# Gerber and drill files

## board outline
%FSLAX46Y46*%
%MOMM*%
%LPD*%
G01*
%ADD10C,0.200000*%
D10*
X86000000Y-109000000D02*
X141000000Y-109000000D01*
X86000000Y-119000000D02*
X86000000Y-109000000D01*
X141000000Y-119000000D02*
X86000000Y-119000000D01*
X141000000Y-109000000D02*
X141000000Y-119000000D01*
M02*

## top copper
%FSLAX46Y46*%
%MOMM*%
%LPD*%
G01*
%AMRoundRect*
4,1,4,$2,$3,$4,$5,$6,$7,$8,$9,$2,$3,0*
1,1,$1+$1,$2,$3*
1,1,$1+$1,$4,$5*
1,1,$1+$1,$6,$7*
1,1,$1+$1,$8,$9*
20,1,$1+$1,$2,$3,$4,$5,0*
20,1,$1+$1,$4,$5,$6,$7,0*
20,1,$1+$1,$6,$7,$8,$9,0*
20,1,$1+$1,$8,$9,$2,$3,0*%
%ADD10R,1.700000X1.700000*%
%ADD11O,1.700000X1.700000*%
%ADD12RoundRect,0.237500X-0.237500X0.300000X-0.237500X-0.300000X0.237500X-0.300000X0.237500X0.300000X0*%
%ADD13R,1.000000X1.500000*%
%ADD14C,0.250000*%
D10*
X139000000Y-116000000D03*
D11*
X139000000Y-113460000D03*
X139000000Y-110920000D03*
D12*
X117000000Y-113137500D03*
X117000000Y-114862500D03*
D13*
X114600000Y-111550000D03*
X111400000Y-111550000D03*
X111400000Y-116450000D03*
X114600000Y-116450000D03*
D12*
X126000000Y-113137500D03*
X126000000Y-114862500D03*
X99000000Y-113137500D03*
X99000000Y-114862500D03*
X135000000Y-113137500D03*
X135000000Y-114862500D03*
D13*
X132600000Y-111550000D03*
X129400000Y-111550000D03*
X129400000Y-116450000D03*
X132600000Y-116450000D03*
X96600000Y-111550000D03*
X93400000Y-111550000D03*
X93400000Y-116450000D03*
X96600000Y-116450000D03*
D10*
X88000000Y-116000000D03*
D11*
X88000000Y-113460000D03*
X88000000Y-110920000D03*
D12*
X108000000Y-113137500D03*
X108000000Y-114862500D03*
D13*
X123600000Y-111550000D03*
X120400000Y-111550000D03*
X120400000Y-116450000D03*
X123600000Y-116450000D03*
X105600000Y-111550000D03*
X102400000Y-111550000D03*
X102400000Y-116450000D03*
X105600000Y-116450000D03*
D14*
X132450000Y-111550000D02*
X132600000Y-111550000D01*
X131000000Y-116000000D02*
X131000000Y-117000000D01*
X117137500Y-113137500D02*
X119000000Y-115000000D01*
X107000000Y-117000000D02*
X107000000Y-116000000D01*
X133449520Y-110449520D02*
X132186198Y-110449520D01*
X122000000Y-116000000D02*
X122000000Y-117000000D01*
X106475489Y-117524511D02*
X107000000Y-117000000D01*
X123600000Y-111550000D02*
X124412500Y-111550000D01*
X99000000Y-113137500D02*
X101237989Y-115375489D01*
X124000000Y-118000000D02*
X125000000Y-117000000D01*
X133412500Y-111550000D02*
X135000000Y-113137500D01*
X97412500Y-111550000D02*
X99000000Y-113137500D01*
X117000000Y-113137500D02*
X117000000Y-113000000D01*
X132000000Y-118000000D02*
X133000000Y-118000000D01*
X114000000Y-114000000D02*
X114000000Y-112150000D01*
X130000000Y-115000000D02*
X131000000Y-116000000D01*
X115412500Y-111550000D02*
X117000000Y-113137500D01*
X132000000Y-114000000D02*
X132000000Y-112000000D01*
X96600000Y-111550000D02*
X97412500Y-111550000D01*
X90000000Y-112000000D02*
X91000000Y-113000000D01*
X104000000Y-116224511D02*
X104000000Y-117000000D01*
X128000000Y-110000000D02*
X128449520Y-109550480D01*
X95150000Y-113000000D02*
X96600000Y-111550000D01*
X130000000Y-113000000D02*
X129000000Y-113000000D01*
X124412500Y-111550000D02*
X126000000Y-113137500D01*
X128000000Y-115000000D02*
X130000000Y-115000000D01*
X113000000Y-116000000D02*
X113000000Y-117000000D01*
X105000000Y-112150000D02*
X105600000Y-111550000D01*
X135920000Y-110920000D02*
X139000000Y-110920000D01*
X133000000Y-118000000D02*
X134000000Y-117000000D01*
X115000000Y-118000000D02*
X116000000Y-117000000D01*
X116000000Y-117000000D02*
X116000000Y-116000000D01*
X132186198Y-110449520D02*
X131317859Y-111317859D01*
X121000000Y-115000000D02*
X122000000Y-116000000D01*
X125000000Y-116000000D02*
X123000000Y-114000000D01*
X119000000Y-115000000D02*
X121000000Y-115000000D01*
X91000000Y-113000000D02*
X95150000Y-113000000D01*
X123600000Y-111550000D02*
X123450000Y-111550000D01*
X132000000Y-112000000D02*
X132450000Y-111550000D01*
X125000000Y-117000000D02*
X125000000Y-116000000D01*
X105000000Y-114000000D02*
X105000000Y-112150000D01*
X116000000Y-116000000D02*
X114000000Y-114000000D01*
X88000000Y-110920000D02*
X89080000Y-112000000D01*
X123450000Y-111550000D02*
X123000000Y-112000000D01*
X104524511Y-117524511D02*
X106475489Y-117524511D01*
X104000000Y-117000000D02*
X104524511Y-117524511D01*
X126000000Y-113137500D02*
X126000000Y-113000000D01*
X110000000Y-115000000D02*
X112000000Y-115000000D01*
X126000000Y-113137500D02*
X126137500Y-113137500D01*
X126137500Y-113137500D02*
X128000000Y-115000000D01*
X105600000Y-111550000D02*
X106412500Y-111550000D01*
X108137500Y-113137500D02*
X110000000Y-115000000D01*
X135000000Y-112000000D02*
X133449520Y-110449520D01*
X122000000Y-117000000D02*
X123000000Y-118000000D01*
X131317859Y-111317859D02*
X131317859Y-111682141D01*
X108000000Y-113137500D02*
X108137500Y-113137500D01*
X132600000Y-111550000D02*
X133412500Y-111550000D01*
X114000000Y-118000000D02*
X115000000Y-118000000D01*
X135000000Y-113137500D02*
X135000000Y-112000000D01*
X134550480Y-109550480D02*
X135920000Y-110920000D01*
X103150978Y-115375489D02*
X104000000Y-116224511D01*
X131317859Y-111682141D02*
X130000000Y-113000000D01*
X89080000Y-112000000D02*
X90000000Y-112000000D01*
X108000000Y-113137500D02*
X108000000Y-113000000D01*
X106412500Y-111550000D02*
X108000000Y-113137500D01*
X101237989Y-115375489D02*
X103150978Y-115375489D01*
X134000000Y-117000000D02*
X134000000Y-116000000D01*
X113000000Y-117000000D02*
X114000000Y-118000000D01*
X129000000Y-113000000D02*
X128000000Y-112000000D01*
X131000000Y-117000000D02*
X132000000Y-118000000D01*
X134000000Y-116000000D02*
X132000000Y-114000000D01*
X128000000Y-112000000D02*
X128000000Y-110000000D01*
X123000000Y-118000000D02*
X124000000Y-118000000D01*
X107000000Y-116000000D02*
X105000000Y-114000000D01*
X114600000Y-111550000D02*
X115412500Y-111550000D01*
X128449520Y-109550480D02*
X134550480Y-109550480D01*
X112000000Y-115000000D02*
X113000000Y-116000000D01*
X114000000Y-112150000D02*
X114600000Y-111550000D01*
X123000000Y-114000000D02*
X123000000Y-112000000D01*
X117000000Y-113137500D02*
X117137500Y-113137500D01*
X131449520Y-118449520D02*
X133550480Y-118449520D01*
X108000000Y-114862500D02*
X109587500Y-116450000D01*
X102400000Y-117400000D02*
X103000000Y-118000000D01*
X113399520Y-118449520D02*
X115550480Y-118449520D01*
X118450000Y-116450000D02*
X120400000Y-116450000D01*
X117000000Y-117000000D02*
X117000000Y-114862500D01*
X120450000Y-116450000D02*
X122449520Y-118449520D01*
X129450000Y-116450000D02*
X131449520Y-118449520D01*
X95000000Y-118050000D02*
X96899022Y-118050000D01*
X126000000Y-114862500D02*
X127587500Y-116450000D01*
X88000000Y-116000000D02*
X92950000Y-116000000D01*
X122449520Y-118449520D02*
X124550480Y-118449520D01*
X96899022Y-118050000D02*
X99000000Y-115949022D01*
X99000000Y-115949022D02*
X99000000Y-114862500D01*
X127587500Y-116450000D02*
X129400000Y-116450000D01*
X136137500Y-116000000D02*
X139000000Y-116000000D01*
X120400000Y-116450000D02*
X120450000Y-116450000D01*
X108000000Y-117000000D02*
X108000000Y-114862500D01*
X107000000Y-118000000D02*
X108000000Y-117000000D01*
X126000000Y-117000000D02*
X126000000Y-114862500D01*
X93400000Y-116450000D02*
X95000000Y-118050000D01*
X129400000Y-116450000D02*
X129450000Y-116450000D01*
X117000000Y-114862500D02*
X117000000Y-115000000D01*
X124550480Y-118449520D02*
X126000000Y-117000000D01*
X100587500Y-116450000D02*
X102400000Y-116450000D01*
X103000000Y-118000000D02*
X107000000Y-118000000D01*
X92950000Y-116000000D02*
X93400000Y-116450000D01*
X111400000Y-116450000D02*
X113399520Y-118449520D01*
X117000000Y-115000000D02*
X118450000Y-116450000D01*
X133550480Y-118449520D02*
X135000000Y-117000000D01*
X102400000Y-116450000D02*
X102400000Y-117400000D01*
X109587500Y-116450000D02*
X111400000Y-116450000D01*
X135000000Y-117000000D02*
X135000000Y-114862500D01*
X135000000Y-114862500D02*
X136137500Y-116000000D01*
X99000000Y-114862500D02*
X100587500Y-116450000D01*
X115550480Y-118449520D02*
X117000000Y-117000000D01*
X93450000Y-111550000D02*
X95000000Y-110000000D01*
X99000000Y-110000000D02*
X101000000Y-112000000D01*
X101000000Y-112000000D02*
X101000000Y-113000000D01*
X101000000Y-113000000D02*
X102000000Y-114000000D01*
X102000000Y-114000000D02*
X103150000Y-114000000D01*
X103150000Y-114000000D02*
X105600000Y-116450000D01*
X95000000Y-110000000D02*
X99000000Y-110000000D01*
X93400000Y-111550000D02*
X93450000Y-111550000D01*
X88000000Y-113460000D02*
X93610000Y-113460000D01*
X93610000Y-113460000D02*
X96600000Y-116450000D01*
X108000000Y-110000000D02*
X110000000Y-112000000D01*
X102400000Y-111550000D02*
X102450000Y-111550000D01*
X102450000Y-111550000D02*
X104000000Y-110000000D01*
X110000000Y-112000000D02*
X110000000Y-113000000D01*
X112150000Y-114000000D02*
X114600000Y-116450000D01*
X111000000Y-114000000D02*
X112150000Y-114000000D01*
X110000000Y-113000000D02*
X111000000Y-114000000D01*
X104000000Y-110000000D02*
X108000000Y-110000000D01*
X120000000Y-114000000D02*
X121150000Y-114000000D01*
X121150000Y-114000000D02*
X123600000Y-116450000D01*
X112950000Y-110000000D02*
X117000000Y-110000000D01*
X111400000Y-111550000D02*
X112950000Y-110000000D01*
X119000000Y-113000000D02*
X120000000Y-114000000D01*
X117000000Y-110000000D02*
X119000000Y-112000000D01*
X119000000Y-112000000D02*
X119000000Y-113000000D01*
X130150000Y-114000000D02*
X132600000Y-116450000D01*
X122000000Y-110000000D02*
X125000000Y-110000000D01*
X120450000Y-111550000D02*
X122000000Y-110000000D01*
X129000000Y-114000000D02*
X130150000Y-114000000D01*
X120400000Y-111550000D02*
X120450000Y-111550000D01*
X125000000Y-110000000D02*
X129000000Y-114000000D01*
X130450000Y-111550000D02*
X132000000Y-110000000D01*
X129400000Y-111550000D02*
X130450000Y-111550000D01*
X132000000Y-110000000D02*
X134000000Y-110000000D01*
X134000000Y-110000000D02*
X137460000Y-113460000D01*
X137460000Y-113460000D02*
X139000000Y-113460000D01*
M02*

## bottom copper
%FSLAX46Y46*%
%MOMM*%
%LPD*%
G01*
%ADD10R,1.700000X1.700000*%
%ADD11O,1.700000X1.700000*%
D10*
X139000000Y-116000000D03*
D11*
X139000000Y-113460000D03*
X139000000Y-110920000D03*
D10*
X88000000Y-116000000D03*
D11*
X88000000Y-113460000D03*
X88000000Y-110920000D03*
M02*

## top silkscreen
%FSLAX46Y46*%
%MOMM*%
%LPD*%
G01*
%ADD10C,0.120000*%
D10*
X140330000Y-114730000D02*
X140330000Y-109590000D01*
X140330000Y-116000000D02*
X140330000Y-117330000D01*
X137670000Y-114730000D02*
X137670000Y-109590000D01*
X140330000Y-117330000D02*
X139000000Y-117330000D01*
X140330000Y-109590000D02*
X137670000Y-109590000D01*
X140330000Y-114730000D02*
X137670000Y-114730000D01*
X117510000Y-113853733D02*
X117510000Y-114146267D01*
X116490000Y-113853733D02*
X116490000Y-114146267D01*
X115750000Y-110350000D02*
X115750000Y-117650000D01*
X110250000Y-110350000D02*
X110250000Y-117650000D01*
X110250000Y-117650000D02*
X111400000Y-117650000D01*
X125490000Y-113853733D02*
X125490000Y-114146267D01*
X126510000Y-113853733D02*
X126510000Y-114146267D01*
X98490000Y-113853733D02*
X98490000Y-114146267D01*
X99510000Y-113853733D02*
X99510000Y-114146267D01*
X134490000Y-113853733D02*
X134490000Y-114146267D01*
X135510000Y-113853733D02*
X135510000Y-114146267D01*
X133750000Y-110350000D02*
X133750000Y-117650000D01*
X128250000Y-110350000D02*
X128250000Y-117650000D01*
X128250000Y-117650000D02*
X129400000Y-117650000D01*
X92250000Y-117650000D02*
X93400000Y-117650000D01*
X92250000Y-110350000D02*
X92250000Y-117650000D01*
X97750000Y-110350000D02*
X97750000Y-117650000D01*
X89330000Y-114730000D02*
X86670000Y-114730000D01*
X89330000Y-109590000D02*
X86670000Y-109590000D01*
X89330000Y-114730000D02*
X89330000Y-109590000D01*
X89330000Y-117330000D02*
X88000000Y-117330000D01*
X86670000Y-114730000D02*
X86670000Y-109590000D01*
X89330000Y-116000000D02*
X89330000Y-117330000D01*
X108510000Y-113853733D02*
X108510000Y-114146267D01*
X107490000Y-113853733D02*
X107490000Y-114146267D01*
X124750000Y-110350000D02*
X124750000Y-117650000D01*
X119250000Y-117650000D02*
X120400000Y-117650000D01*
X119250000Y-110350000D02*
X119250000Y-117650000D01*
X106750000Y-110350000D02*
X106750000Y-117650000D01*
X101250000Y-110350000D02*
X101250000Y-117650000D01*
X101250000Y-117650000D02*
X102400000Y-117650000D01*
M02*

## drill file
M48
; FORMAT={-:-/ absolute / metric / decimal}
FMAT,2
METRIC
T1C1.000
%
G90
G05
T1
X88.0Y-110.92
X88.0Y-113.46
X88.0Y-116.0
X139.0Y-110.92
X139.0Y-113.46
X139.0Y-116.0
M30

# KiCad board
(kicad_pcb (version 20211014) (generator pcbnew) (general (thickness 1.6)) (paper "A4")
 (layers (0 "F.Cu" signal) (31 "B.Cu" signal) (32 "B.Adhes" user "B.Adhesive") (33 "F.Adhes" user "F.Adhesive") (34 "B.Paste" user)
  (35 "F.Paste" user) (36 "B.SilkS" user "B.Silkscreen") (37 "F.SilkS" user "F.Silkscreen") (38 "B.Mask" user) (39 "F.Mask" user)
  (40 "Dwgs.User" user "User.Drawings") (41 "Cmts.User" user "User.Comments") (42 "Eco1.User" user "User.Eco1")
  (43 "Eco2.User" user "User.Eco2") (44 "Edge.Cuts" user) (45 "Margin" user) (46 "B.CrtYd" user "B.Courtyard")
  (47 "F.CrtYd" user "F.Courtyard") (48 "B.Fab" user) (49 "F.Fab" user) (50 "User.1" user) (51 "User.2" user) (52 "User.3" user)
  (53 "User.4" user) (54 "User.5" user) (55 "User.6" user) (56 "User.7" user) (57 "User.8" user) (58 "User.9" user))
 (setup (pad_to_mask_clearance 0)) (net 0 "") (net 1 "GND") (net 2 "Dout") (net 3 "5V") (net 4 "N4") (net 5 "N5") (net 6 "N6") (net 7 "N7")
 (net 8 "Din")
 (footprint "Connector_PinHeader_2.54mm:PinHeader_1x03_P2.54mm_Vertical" (layer "F.Cu") (at 139 116 180)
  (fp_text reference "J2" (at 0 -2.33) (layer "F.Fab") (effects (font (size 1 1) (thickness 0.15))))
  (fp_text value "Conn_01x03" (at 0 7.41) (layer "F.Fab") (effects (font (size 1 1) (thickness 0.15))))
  (fp_line (start -1.33 1.27) (end -1.33 6.41) (layer "F.SilkS") (width 0.12))
  (fp_line (start -1.33 0) (end -1.33 -1.33) (layer "F.SilkS") (width 0.12))
  (fp_line (start 1.33 1.27) (end 1.33 6.41) (layer "F.SilkS") (width 0.12))
  (fp_line (start -1.33 -1.33) (end 0 -1.33) (layer "F.SilkS") (width 0.12))
  (fp_line (start -1.33 6.41) (end 1.33 6.41) (layer "F.SilkS") (width 0.12))
  (fp_line (start -1.33 1.27) (end 1.33 1.27) (layer "F.SilkS") (width 0.12))
  (pad "1" thru_hole rect (at 0 0 180) (size 1.7 1.7) (drill 1) (layers *.Cu *.Mask) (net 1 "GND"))
  (pad "2" thru_hole oval (at 0 2.54 180) (size 1.7 1.7) (drill 1) (layers *.Cu *.Mask) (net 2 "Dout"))
  (pad "3" thru_hole oval (at 0 5.08 180) (size 1.7 1.7) (drill 1) (layers *.Cu *.Mask) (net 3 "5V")))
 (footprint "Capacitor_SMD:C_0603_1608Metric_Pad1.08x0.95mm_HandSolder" (layer "F.Cu") (at 117 114 -90)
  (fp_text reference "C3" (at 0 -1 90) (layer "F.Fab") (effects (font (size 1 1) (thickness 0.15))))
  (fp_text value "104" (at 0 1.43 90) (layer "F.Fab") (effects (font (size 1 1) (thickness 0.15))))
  (fp_line (start -0.146267 -0.51) (end 0.146267 -0.51) (layer "F.SilkS") (width 0.12))
  (fp_line (start -0.146267 0.51) (end 0.146267 0.51) (layer "F.SilkS") (width 0.12))
  (pad "1" smd roundrect (at -0.8625 0 270) (size 1.075 0.95) (layers "F.Cu" "F.Paste" "F.Mask") (roundrect_rratio 0.25) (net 3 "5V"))
  (pad "2" smd roundrect (at 0.8625 0 270) (size 1.075 0.95) (layers "F.Cu" "F.Paste" "F.Mask") (roundrect_rratio 0.25) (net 1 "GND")))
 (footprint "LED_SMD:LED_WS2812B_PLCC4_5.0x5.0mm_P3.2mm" (layer "F.Cu") (at 113 114 -90)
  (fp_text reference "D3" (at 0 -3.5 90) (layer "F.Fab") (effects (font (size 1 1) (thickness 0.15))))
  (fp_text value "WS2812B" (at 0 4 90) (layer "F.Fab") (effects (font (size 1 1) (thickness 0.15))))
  (fp_line (start -3.65 -2.75) (end 3.65 -2.75) (layer "F.SilkS") (width 0.12))
  (fp_line (start -3.65 2.75) (end 3.65 2.75) (layer "F.SilkS") (width 0.12))
  (fp_line (start 3.65 2.75) (end 3.65 1.6) (layer "F.SilkS") (width 0.12))
  (pad "1" smd rect (at -2.45 -1.6 270) (size 1.5 1) (layers "F.Cu" "F.Paste" "F.Mask") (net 3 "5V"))
  (pad "2" smd rect (at -2.45 1.6 270) (size 1.5 1) (layers "F.Cu" "F.Paste" "F.Mask") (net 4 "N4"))
  (pad "3" smd rect (at 2.45 1.6 270) (size 1.5 1) (layers "F.Cu" "F.Paste" "F.Mask") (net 1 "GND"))
  (pad "4" smd rect (at 2.45 -1.6 270) (size 1.5 1) (layers "F.Cu" "F.Paste" "F.Mask") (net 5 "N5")))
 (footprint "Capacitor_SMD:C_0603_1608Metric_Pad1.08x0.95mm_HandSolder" (layer "F.Cu") (at 126 114 -90)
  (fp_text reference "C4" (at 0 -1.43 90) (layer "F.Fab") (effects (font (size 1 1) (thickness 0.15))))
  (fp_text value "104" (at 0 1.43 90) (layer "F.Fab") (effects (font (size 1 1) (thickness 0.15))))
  (fp_line (start -0.146267 0.51) (end 0.146267 0.51) (layer "F.SilkS") (width 0.12))
  (fp_line (start -0.146267 -0.51) (end 0.146267 -0.51) (layer "F.SilkS") (width 0.12))
  (pad "1" smd roundrect (at -0.8625 0 270) (size 1.075 0.95) (layers "F.Cu" "F.Paste" "F.Mask") (roundrect_rratio 0.25) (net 3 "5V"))
  (pad "2" smd roundrect (at 0.8625 0 270) (size 1.075 0.95) (layers "F.Cu" "F.Paste" "F.Mask") (roundrect_rratio 0.25) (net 1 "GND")))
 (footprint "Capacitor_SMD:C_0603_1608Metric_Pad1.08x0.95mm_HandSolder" (layer "F.Cu") (at 99 114 -90)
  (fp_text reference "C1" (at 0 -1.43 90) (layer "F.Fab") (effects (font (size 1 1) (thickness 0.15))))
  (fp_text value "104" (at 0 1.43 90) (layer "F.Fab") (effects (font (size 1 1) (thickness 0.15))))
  (fp_line (start -0.146267 0.51) (end 0.146267 0.51) (layer "F.SilkS") (width 0.12))
  (fp_line (start -0.146267 -0.51) (end 0.146267 -0.51) (layer "F.SilkS") (width 0.12))
  (pad "1" smd roundrect (at -0.8625 0 270) (size 1.075 0.95) (layers "F.Cu" "F.Paste" "F.Mask") (roundrect_rratio 0.25) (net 3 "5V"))
  (pad "2" smd roundrect (at 0.8625 0 270) (size 1.075 0.95) (layers "F.Cu" "F.Paste" "F.Mask") (roundrect_rratio 0.25) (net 1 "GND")))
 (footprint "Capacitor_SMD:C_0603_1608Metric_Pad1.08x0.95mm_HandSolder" (layer "F.Cu") (at 135 114 -90)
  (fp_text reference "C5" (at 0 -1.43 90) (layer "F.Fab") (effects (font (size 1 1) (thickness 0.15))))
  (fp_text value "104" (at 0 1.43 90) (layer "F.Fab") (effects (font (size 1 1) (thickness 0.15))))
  (fp_line (start -0.146267 0.51) (end 0.146267 0.51) (layer "F.SilkS") (width 0.12))
  (fp_line (start -0.146267 -0.51) (end 0.146267 -0.51) (layer "F.SilkS") (width 0.12))
  (pad "1" smd roundrect (at -0.8625 0 270) (size 1.075 0.95) (layers "F.Cu" "F.Paste" "F.Mask") (roundrect_rratio 0.25) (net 3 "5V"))
  (pad "2" smd roundrect (at 0.8625 0 270) (size 1.075 0.95) (layers "F.Cu" "F.Paste" "F.Mask") (roundrect_rratio 0.25) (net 1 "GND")))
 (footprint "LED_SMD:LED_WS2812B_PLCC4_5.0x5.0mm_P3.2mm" (layer "F.Cu") (at 131 114 -90)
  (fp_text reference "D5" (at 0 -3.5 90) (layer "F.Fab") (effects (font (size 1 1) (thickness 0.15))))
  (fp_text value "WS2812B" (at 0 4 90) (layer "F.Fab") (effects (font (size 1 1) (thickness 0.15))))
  (fp_line (start -3.65 -2.75) (end 3.65 -2.75) (layer "F.SilkS") (width 0.12))
  (fp_line (start -3.65 2.75) (end 3.65 2.75) (layer "F.SilkS") (width 0.12))
  (fp_line (start 3.65 2.75) (end 3.65 1.6) (layer "F.SilkS") (width 0.12))
  (pad "1" smd rect (at -2.45 -1.6 270) (size 1.5 1) (layers "F.Cu" "F.Paste" "F.Mask") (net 3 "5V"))
  (pad "2" smd rect (at -2.45 1.6 270) (size 1.5 1) (layers "F.Cu" "F.Paste" "F.Mask") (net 2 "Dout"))
  (pad "3" smd rect (at 2.45 1.6 270) (size 1.5 1) (layers "F.Cu" "F.Paste" "F.Mask") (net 1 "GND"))
  (pad "4" smd rect (at 2.45 -1.6 270) (size 1.5 1) (layers "F.Cu" "F.Paste" "F.Mask") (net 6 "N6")))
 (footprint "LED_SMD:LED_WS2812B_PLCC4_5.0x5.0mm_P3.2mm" (layer "F.Cu") (at 95 114 -90)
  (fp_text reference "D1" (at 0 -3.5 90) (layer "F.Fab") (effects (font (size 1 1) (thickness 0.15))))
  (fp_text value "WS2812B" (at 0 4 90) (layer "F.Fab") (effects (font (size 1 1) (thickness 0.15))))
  (fp_line (start 3.65 2.75) (end 3.65 1.6) (layer "F.SilkS") (width 0.12))
  (fp_line (start -3.65 2.75) (end 3.65 2.75) (layer "F.SilkS") (width 0.12))
  (fp_line (start -3.65 -2.75) (end 3.65 -2.75) (layer "F.SilkS") (width 0.12))
  (pad "1" smd rect (at -2.45 -1.6 270) (size 1.5 1) (layers "F.Cu" "F.Paste" "F.Mask") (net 3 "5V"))
  (pad "2" smd rect (at -2.45 1.6 270) (size 1.5 1) (layers "F.Cu" "F.Paste" "F.Mask") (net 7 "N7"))
  (pad "3" smd rect (at 2.45 1.6 270) (size 1.5 1) (layers "F.Cu" "F.Paste" "F.Mask") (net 1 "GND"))
  (pad "4" smd rect (at 2.45 -1.6 270) (size 1.5 1) (layers "F.Cu" "F.Paste" "F.Mask") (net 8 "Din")))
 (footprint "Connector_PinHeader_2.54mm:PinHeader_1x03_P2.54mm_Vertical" (layer "F.Cu") (at 88 116 180)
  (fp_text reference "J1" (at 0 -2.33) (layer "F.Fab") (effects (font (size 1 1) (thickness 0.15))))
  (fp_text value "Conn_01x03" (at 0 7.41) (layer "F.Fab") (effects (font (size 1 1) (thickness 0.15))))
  (fp_line (start -1.33 1.27) (end 1.33 1.27) (layer "F.SilkS") (width 0.12))
  (fp_line (start -1.33 6.41) (end 1.33 6.41) (layer "F.SilkS") (width 0.12))
  (fp_line (start -1.33 1.27) (end -1.33 6.41) (layer "F.SilkS") (width 0.12))
  (fp_line (start -1.33 -1.33) (end 0 -1.33) (layer "F.SilkS") (width 0.12))
  (fp_line (start 1.33 1.27) (end 1.33 6.41) (layer "F.SilkS") (width 0.12))
  (fp_line (start -1.33 0) (end -1.33 -1.33) (layer "F.SilkS") (width 0.12))
  (pad "1" thru_hole rect (at 0 0 180) (size 1.7 1.7) (drill 1) (layers *.Cu *.Mask) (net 1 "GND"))
  (pad "2" thru_hole oval (at 0 2.54 180) (size 1.7 1.7) (drill 1) (layers *.Cu *.Mask) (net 8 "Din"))
  (pad "3" thru_hole oval (at 0 5.08 180) (size 1.7 1.7) (drill 1) (layers *.Cu *.Mask) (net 3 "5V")))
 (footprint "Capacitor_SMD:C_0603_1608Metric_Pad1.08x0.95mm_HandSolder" (layer "F.Cu") (at 108 114 -90)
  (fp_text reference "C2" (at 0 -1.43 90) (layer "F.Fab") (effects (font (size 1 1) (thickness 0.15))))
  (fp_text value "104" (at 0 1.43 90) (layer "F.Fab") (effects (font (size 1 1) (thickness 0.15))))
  (fp_line (start -0.146267 -0.51) (end 0.146267 -0.51) (layer "F.SilkS") (width 0.12))
  (fp_line (start -0.146267 0.51) (end 0.146267 0.51) (layer "F.SilkS") (width 0.12))
  (pad "1" smd roundrect (at -0.8625 0 270) (size 1.075 0.95) (layers "F.Cu" "F.Paste" "F.Mask") (roundrect_rratio 0.25) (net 3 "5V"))
  (pad "2" smd roundrect (at 0.8625 0 270) (size 1.075 0.95) (layers "F.Cu" "F.Paste" "F.Mask") (roundrect_rratio 0.25) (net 1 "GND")))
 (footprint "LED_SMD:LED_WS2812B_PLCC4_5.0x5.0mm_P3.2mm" (layer "F.Cu") (at 122 114 -90)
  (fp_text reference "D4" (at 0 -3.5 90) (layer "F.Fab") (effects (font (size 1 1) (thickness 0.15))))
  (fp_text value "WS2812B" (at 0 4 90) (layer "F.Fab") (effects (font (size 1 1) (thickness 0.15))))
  (fp_line (start -3.65 -2.75) (end 3.65 -2.75) (layer "F.SilkS") (width 0.12))
  (fp_line (start 3.65 2.75) (end 3.65 1.6) (layer "F.SilkS") (width 0.12))
  (fp_line (start -3.65 2.75) (end 3.65 2.75) (layer "F.SilkS") (width 0.12))
  (pad "1" smd rect (at -2.45 -1.6 270) (size 1.5 1) (layers "F.Cu" "F.Paste" "F.Mask") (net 3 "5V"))
  (pad "2" smd rect (at -2.45 1.6 270) (size 1.5 1) (layers "F.Cu" "F.Paste" "F.Mask") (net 6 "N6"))
  (pad "3" smd rect (at 2.45 1.6 270) (size 1.5 1) (layers "F.Cu" "F.Paste" "F.Mask") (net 1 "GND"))
  (pad "4" smd rect (at 2.45 -1.6 270) (size 1.5 1) (layers "F.Cu" "F.Paste" "F.Mask") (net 4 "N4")))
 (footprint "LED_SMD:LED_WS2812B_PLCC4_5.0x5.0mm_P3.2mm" (layer "F.Cu") (at 104 114 -90)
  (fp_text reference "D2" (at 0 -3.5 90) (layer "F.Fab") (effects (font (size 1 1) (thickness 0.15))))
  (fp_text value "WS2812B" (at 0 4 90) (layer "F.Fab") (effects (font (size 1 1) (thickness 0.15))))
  (fp_line (start -3.65 -2.75) (end 3.65 -2.75) (layer "F.SilkS") (width 0.12))
  (fp_line (start -3.65 2.75) (end 3.65 2.75) (layer "F.SilkS") (width 0.12))
  (fp_line (start 3.65 2.75) (end 3.65 1.6) (layer "F.SilkS") (width 0.12))
  (pad "1" smd rect (at -2.45 -1.6 270) (size 1.5 1) (layers "F.Cu" "F.Paste" "F.Mask") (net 3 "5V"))
  (pad "2" smd rect (at -2.45 1.6 270) (size 1.5 1) (layers "F.Cu" "F.Paste" "F.Mask") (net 5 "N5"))
  (pad "3" smd rect (at 2.45 1.6 270) (size 1.5 1) (layers "F.Cu" "F.Paste" "F.Mask") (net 1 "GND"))
  (pad "4" smd rect (at 2.45 -1.6 270) (size 1.5 1) (layers "F.Cu" "F.Paste" "F.Mask") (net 7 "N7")))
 (gr_line (start 86 109) (end 141 109) (layer "Edge.Cuts") (width 0.2))
 (gr_line (start 86 119) (end 86 109) (layer "Edge.Cuts") (width 0.2))
 (gr_line (start 141 119) (end 86 119) (layer "Edge.Cuts") (width 0.2))
 (gr_line (start 141 109) (end 141 119) (layer "Edge.Cuts") (width 0.2))
 (segment (start 132.45 111.55) (end 132.6 111.55) (width 0.25) (layer "F.Cu") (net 3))
 (segment (start 131 116) (end 131 117) (width 0.25) (layer "F.Cu") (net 3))
 (segment (start 117.1375 113.1375) (end 119 115) (width 0.25) (layer "F.Cu") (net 3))
 (segment (start 107 117) (end 107 116) (width 0.25) (layer "F.Cu") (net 3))
 (segment (start 133.44952 110.44952) (end 132.186198 110.44952) (width 0.25) (layer "F.Cu") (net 3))
 (segment (start 122 116) (end 122 117) (width 0.25) (layer "F.Cu") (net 3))
 (segment (start 106.475489 117.524511) (end 107 117) (width 0.25) (layer "F.Cu") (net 3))
 (segment (start 123.6 111.55) (end 124.4125 111.55) (width 0.25) (layer "F.Cu") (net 3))
 (segment (start 99 113.1375) (end 101.237989 115.375489) (width 0.25) (layer "F.Cu") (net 3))
 (segment (start 124 118) (end 125 117) (width 0.25) (layer "F.Cu") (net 3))
 (segment (start 133.4125 111.55) (end 135 113.1375) (width 0.25) (layer "F.Cu") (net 3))
 (segment (start 97.4125 111.55) (end 99 113.1375) (width 0.25) (layer "F.Cu") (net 3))
 (segment (start 117 113.1375) (end 117 113) (width 0.25) (layer "F.Cu") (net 3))
 (segment (start 132 118) (end 133 118) (width 0.25) (layer "F.Cu") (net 3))
 (segment (start 114 114) (end 114 112.15) (width 0.25) (layer "F.Cu") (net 3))
 (segment (start 130 115) (end 131 116) (width 0.25) (layer "F.Cu") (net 3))
 (segment (start 115.4125 111.55) (end 117 113.1375) (width 0.25) (layer "F.Cu") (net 3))
 (segment (start 132 114) (end 132 112) (width 0.25) (layer "F.Cu") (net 3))
 (segment (start 96.6 111.55) (end 97.4125 111.55) (width 0.25) (layer "F.Cu") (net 3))
 (segment (start 90 112) (end 91 113) (width 0.25) (layer "F.Cu") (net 3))
 (segment (start 104 116.224511) (end 104 117) (width 0.25) (layer "F.Cu") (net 3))
 (segment (start 128 110) (end 128.44952 109.55048) (width 0.25) (layer "F.Cu") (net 3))
 (segment (start 95.15 113) (end 96.6 111.55) (width 0.25) (layer "F.Cu") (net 3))
 (segment (start 130 113) (end 129 113) (width 0.25) (layer "F.Cu") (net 3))
 (segment (start 124.4125 111.55) (end 126 113.1375) (width 0.25) (layer "F.Cu") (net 3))
 (segment (start 128 115) (end 130 115) (width 0.25) (layer "F.Cu") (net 3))
 (segment (start 113 116) (end 113 117) (width 0.25) (layer "F.Cu") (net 3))
 (segment (start 105 112.15) (end 105.6 111.55) (width 0.25) (layer "F.Cu") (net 3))
 (segment (start 135.92 110.92) (end 139 110.92) (width 0.25) (layer "F.Cu") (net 3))
 (segment (start 133 118) (end 134 117) (width 0.25) (layer "F.Cu") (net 3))
 (segment (start 115 118) (end 116 117) (width 0.25) (layer "F.Cu") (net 3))
 (segment (start 116 117) (end 116 116) (width 0.25) (layer "F.Cu") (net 3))
 (segment (start 132.186198 110.44952) (end 131.317859 111.317859) (width 0.25) (layer "F.Cu") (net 3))
 (segment (start 121 115) (end 122 116) (width 0.25) (layer "F.Cu") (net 3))
 (segment (start 125 116) (end 123 114) (width 0.25) (layer "F.Cu") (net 3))
 (segment (start 119 115) (end 121 115) (width 0.25) (layer "F.Cu") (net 3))
 (segment (start 91 113) (end 95.15 113) (width 0.25) (layer "F.Cu") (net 3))
 (segment (start 123.6 111.55) (end 123.45 111.55) (width 0.25) (layer "F.Cu") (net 3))
 (segment (start 132 112) (end 132.45 111.55) (width 0.25) (layer "F.Cu") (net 3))
 (segment (start 125 117) (end 125 116) (width 0.25) (layer "F.Cu") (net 3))
 (segment (start 105 114) (end 105 112.15) (width 0.25) (layer "F.Cu") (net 3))
 (segment (start 116 116) (end 114 114) (width 0.25) (layer "F.Cu") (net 3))
 (segment (start 88 110.92) (end 89.08 112) (width 0.25) (layer "F.Cu") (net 3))
 (segment (start 123.45 111.55) (end 123 112) (width 0.25) (layer "F.Cu") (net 3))
 (segment (start 104.524511 117.524511) (end 106.475489 117.524511) (width 0.25) (layer "F.Cu") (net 3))
 (segment (start 104 117) (end 104.524511 117.524511) (width 0.25) (layer "F.Cu") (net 3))
 (segment (start 126 113.1375) (end 126 113) (width 0.25) (layer "F.Cu") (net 3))
 (segment (start 110 115) (end 112 115) (width 0.25) (layer "F.Cu") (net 3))
 (segment (start 126 113.1375) (end 126.1375 113.1375) (width 0.25) (layer "F.Cu") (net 3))
 (segment (start 126.1375 113.1375) (end 128 115) (width 0.25) (layer "F.Cu") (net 3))
 (segment (start 105.6 111.55) (end 106.4125 111.55) (width 0.25) (layer "F.Cu") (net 3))
 (segment (start 108.1375 113.1375) (end 110 115) (width 0.25) (layer "F.Cu") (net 3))
 (segment (start 135 112) (end 133.44952 110.44952) (width 0.25) (layer "F.Cu") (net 3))
 (segment (start 122 117) (end 123 118) (width 0.25) (layer "F.Cu") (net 3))
 (segment (start 131.317859 111.317859) (end 131.317859 111.682141) (width 0.25) (layer "F.Cu") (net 3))
 (segment (start 108 113.1375) (end 108.1375 113.1375) (width 0.25) (layer "F.Cu") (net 3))
 (segment (start 132.6 111.55) (end 133.4125 111.55) (width 0.25) (layer "F.Cu") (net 3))
 (segment (start 114 118) (end 115 118) (width 0.25) (layer "F.Cu") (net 3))
 (segment (start 135 113.1375) (end 135 112) (width 0.25) (layer "F.Cu") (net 3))
 (segment (start 134.55048 109.55048) (end 135.92 110.92) (width 0.25) (layer "F.Cu") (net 3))
 (segment (start 103.150978 115.375489) (end 104 116.224511) (width 0.25) (layer "F.Cu") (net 3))
 (segment (start 131.317859 111.682141) (end 130 113) (width 0.25) (layer "F.Cu") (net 3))
 (segment (start 89.08 112) (end 90 112) (width 0.25) (layer "F.Cu") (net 3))
 (segment (start 108 113.1375) (end 108 113) (width 0.25) (layer "F.Cu") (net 3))
 (segment (start 106.4125 111.55) (end 108 113.1375) (width 0.25) (layer "F.Cu") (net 3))
 (segment (start 101.237989 115.375489) (end 103.150978 115.375489) (width 0.25) (layer "F.Cu") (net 3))
 (segment (start 134 117) (end 134 116) (width 0.25) (layer "F.Cu") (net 3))
 (segment (start 113 117) (end 114 118) (width 0.25) (layer "F.Cu") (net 3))
 (segment (start 129 113) (end 128 112) (width 0.25) (layer "F.Cu") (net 3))
 (segment (start 131 117) (end 132 118) (width 0.25) (layer "F.Cu") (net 3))
 (segment (start 134 116) (end 132 114) (width 0.25) (layer "F.Cu") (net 3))
 (segment (start 128 112) (end 128 110) (width 0.25) (layer "F.Cu") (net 3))
 (segment (start 123 118) (end 124 118) (width 0.25) (layer "F.Cu") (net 3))
 (segment (start 107 116) (end 105 114) (width 0.25) (layer "F.Cu") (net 3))
 (segment (start 114.6 111.55) (end 115.4125 111.55) (width 0.25) (layer "F.Cu") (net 3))
 (segment (start 128.44952 109.55048) (end 134.55048 109.55048) (width 0.25) (layer "F.Cu") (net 3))
 (segment (start 112 115) (end 113 116) (width 0.25) (layer "F.Cu") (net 3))
 (segment (start 114 112.15) (end 114.6 111.55) (width 0.25) (layer "F.Cu") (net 3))
 (segment (start 123 114) (end 123 112) (width 0.25) (layer "F.Cu") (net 3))
 (segment (start 117 113.1375) (end 117.1375 113.1375) (width 0.25) (layer "F.Cu") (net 3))
 (segment (start 131.44952 118.44952) (end 133.55048 118.44952) (width 0.25) (layer "F.Cu") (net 1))
 (segment (start 108 114.8625) (end 109.5875 116.45) (width 0.25) (layer "F.Cu") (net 1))
 (segment (start 102.4 117.4) (end 103 118) (width 0.25) (layer "F.Cu") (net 1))
 (segment (start 113.39952 118.44952) (end 115.55048 118.44952) (width 0.25) (layer "F.Cu") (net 1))
 (segment (start 118.45 116.45) (end 120.4 116.45) (width 0.25) (layer "F.Cu") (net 1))
 (segment (start 117 117) (end 117 114.8625) (width 0.25) (layer "F.Cu") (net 1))
 (segment (start 120.45 116.45) (end 122.44952 118.44952) (width 0.25) (layer "F.Cu") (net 1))
 (segment (start 129.45 116.45) (end 131.44952 118.44952) (width 0.25) (layer "F.Cu") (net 1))
 (segment (start 95 118.05) (end 96.899022 118.05) (width 0.25) (layer "F.Cu") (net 1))
 (segment (start 126 114.8625) (end 127.5875 116.45) (width 0.25) (layer "F.Cu") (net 1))
 (segment (start 88 116) (end 92.95 116) (width 0.25) (layer "F.Cu") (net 1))
 (segment (start 122.44952 118.44952) (end 124.55048 118.44952) (width 0.25) (layer "F.Cu") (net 1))
 (segment (start 96.899022 118.05) (end 99 115.949022) (width 0.25) (layer "F.Cu") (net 1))
 (segment (start 99 115.949022) (end 99 114.8625) (width 0.25) (layer "F.Cu") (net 1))
 (segment (start 127.5875 116.45) (end 129.4 116.45) (width 0.25) (layer "F.Cu") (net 1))
 (segment (start 136.1375 116) (end 139 116) (width 0.25) (layer "F.Cu") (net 1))
 (segment (start 120.4 116.45) (end 120.45 116.45) (width 0.25) (layer "F.Cu") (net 1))
 (segment (start 108 117) (end 108 114.8625) (width 0.25) (layer "F.Cu") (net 1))
 (segment (start 107 118) (end 108 117) (width 0.25) (layer "F.Cu") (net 1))
 (segment (start 126 117) (end 126 114.8625) (width 0.25) (layer "F.Cu") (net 1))
 (segment (start 93.4 116.45) (end 95 118.05) (width 0.25) (layer "F.Cu") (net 1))
 (segment (start 129.4 116.45) (end 129.45 116.45) (width 0.25) (layer "F.Cu") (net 1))
 (segment (start 117 114.8625) (end 117 115) (width 0.25) (layer "F.Cu") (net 1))
 (segment (start 124.55048 118.44952) (end 126 117) (width 0.25) (layer "F.Cu") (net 1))
 (segment (start 100.5875 116.45) (end 102.4 116.45) (width 0.25) (layer "F.Cu") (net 1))
 (segment (start 103 118) (end 107 118) (width 0.25) (layer "F.Cu") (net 1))
 (segment (start 92.95 116) (end 93.4 116.45) (width 0.25) (layer "F.Cu") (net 1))
 (segment (start 111.4 116.45) (end 113.39952 118.44952) (width 0.25) (layer "F.Cu") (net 1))
 (segment (start 117 115) (end 118.45 116.45) (width 0.25) (layer "F.Cu") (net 1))
 (segment (start 133.55048 118.44952) (end 135 117) (width 0.25) (layer "F.Cu") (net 1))
 (segment (start 102.4 116.45) (end 102.4 117.4) (width 0.25) (layer "F.Cu") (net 1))
 (segment (start 109.5875 116.45) (end 111.4 116.45) (width 0.25) (layer "F.Cu") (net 1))
 (segment (start 135 117) (end 135 114.8625) (width 0.25) (layer "F.Cu") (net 1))
 (segment (start 135 114.8625) (end 136.1375 116) (width 0.25) (layer "F.Cu") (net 1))
 (segment (start 99 114.8625) (end 100.5875 116.45) (width 0.25) (layer "F.Cu") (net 1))
 (segment (start 115.55048 118.44952) (end 117 117) (width 0.25) (layer "F.Cu") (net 1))
 (segment (start 93.45 111.55) (end 95 110) (width 0.25) (layer "F.Cu") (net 7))
 (segment (start 99 110) (end 101 112) (width 0.25) (layer "F.Cu") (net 7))
 (segment (start 101 112) (end 101 113) (width 0.25) (layer "F.Cu") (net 7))
 (segment (start 101 113) (end 102 114) (width 0.25) (layer "F.Cu") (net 7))
 (segment (start 102 114) (end 103.15 114) (width 0.25) (layer "F.Cu") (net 7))
 (segment (start 103.15 114) (end 105.6 116.45) (width 0.25) (layer "F.Cu") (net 7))
 (segment (start 95 110) (end 99 110) (width 0.25) (layer "F.Cu") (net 7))
 (segment (start 93.4 111.55) (end 93.45 111.55) (width 0.25) (layer "F.Cu") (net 7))
 (segment (start 88 113.46) (end 93.61 113.46) (width 0.25) (layer "F.Cu") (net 8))
 (segment (start 93.61 113.46) (end 96.6 116.45) (width 0.25) (layer "F.Cu") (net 8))
 (segment (start 108 110) (end 110 112) (width 0.25) (layer "F.Cu") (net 5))
 (segment (start 102.4 111.55) (end 102.45 111.55) (width 0.25) (layer "F.Cu") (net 5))
 (segment (start 102.45 111.55) (end 104 110) (width 0.25) (layer "F.Cu") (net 5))
 (segment (start 110 112) (end 110 113) (width 0.25) (layer "F.Cu") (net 5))
 (segment (start 112.15 114) (end 114.6 116.45) (width 0.25) (layer "F.Cu") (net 5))
 (segment (start 111 114) (end 112.15 114) (width 0.25) (layer "F.Cu") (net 5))
 (segment (start 110 113) (end 111 114) (width 0.25) (layer "F.Cu") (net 5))
 (segment (start 104 110) (end 108 110) (width 0.25) (layer "F.Cu") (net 5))
 (segment (start 120 114) (end 121.15 114) (width 0.25) (layer "F.Cu") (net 4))
 (segment (start 121.15 114) (end 123.6 116.45) (width 0.25) (layer "F.Cu") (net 4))
 (segment (start 112.95 110) (end 117 110) (width 0.25) (layer "F.Cu") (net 4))
 (segment (start 111.4 111.55) (end 112.95 110) (width 0.25) (layer "F.Cu") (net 4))
 (segment (start 119 113) (end 120 114) (width 0.25) (layer "F.Cu") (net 4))
 (segment (start 117 110) (end 119 112) (width 0.25) (layer "F.Cu") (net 4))
 (segment (start 119 112) (end 119 113) (width 0.25) (layer "F.Cu") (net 4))
 (segment (start 130.15 114) (end 132.6 116.45) (width 0.25) (layer "F.Cu") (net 6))
 (segment (start 122 110) (end 125 110) (width 0.25) (layer "F.Cu") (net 6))
 (segment (start 120.45 111.55) (end 122 110) (width 0.25) (layer "F.Cu") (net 6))
 (segment (start 129 114) (end 130.15 114) (width 0.25) (layer "F.Cu") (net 6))
 (segment (start 120.4 111.55) (end 120.45 111.55) (width 0.25) (layer "F.Cu") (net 6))
 (segment (start 125 110) (end 129 114) (width 0.25) (layer "F.Cu") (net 6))
 (segment (start 130.45 111.55) (end 132 110) (width 0.25) (layer "F.Cu") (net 2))
 (segment (start 129.4 111.55) (end 130.45 111.55) (width 0.25) (layer "F.Cu") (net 2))
 (segment (start 132 110) (end 134 110) (width 0.25) (layer "F.Cu") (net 2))
 (segment (start 134 110) (end 137.46 113.46) (width 0.25) (layer "F.Cu") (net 2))
 (segment (start 137.46 113.46) (end 139 113.46) (width 0.25) (layer "F.Cu") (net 2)))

